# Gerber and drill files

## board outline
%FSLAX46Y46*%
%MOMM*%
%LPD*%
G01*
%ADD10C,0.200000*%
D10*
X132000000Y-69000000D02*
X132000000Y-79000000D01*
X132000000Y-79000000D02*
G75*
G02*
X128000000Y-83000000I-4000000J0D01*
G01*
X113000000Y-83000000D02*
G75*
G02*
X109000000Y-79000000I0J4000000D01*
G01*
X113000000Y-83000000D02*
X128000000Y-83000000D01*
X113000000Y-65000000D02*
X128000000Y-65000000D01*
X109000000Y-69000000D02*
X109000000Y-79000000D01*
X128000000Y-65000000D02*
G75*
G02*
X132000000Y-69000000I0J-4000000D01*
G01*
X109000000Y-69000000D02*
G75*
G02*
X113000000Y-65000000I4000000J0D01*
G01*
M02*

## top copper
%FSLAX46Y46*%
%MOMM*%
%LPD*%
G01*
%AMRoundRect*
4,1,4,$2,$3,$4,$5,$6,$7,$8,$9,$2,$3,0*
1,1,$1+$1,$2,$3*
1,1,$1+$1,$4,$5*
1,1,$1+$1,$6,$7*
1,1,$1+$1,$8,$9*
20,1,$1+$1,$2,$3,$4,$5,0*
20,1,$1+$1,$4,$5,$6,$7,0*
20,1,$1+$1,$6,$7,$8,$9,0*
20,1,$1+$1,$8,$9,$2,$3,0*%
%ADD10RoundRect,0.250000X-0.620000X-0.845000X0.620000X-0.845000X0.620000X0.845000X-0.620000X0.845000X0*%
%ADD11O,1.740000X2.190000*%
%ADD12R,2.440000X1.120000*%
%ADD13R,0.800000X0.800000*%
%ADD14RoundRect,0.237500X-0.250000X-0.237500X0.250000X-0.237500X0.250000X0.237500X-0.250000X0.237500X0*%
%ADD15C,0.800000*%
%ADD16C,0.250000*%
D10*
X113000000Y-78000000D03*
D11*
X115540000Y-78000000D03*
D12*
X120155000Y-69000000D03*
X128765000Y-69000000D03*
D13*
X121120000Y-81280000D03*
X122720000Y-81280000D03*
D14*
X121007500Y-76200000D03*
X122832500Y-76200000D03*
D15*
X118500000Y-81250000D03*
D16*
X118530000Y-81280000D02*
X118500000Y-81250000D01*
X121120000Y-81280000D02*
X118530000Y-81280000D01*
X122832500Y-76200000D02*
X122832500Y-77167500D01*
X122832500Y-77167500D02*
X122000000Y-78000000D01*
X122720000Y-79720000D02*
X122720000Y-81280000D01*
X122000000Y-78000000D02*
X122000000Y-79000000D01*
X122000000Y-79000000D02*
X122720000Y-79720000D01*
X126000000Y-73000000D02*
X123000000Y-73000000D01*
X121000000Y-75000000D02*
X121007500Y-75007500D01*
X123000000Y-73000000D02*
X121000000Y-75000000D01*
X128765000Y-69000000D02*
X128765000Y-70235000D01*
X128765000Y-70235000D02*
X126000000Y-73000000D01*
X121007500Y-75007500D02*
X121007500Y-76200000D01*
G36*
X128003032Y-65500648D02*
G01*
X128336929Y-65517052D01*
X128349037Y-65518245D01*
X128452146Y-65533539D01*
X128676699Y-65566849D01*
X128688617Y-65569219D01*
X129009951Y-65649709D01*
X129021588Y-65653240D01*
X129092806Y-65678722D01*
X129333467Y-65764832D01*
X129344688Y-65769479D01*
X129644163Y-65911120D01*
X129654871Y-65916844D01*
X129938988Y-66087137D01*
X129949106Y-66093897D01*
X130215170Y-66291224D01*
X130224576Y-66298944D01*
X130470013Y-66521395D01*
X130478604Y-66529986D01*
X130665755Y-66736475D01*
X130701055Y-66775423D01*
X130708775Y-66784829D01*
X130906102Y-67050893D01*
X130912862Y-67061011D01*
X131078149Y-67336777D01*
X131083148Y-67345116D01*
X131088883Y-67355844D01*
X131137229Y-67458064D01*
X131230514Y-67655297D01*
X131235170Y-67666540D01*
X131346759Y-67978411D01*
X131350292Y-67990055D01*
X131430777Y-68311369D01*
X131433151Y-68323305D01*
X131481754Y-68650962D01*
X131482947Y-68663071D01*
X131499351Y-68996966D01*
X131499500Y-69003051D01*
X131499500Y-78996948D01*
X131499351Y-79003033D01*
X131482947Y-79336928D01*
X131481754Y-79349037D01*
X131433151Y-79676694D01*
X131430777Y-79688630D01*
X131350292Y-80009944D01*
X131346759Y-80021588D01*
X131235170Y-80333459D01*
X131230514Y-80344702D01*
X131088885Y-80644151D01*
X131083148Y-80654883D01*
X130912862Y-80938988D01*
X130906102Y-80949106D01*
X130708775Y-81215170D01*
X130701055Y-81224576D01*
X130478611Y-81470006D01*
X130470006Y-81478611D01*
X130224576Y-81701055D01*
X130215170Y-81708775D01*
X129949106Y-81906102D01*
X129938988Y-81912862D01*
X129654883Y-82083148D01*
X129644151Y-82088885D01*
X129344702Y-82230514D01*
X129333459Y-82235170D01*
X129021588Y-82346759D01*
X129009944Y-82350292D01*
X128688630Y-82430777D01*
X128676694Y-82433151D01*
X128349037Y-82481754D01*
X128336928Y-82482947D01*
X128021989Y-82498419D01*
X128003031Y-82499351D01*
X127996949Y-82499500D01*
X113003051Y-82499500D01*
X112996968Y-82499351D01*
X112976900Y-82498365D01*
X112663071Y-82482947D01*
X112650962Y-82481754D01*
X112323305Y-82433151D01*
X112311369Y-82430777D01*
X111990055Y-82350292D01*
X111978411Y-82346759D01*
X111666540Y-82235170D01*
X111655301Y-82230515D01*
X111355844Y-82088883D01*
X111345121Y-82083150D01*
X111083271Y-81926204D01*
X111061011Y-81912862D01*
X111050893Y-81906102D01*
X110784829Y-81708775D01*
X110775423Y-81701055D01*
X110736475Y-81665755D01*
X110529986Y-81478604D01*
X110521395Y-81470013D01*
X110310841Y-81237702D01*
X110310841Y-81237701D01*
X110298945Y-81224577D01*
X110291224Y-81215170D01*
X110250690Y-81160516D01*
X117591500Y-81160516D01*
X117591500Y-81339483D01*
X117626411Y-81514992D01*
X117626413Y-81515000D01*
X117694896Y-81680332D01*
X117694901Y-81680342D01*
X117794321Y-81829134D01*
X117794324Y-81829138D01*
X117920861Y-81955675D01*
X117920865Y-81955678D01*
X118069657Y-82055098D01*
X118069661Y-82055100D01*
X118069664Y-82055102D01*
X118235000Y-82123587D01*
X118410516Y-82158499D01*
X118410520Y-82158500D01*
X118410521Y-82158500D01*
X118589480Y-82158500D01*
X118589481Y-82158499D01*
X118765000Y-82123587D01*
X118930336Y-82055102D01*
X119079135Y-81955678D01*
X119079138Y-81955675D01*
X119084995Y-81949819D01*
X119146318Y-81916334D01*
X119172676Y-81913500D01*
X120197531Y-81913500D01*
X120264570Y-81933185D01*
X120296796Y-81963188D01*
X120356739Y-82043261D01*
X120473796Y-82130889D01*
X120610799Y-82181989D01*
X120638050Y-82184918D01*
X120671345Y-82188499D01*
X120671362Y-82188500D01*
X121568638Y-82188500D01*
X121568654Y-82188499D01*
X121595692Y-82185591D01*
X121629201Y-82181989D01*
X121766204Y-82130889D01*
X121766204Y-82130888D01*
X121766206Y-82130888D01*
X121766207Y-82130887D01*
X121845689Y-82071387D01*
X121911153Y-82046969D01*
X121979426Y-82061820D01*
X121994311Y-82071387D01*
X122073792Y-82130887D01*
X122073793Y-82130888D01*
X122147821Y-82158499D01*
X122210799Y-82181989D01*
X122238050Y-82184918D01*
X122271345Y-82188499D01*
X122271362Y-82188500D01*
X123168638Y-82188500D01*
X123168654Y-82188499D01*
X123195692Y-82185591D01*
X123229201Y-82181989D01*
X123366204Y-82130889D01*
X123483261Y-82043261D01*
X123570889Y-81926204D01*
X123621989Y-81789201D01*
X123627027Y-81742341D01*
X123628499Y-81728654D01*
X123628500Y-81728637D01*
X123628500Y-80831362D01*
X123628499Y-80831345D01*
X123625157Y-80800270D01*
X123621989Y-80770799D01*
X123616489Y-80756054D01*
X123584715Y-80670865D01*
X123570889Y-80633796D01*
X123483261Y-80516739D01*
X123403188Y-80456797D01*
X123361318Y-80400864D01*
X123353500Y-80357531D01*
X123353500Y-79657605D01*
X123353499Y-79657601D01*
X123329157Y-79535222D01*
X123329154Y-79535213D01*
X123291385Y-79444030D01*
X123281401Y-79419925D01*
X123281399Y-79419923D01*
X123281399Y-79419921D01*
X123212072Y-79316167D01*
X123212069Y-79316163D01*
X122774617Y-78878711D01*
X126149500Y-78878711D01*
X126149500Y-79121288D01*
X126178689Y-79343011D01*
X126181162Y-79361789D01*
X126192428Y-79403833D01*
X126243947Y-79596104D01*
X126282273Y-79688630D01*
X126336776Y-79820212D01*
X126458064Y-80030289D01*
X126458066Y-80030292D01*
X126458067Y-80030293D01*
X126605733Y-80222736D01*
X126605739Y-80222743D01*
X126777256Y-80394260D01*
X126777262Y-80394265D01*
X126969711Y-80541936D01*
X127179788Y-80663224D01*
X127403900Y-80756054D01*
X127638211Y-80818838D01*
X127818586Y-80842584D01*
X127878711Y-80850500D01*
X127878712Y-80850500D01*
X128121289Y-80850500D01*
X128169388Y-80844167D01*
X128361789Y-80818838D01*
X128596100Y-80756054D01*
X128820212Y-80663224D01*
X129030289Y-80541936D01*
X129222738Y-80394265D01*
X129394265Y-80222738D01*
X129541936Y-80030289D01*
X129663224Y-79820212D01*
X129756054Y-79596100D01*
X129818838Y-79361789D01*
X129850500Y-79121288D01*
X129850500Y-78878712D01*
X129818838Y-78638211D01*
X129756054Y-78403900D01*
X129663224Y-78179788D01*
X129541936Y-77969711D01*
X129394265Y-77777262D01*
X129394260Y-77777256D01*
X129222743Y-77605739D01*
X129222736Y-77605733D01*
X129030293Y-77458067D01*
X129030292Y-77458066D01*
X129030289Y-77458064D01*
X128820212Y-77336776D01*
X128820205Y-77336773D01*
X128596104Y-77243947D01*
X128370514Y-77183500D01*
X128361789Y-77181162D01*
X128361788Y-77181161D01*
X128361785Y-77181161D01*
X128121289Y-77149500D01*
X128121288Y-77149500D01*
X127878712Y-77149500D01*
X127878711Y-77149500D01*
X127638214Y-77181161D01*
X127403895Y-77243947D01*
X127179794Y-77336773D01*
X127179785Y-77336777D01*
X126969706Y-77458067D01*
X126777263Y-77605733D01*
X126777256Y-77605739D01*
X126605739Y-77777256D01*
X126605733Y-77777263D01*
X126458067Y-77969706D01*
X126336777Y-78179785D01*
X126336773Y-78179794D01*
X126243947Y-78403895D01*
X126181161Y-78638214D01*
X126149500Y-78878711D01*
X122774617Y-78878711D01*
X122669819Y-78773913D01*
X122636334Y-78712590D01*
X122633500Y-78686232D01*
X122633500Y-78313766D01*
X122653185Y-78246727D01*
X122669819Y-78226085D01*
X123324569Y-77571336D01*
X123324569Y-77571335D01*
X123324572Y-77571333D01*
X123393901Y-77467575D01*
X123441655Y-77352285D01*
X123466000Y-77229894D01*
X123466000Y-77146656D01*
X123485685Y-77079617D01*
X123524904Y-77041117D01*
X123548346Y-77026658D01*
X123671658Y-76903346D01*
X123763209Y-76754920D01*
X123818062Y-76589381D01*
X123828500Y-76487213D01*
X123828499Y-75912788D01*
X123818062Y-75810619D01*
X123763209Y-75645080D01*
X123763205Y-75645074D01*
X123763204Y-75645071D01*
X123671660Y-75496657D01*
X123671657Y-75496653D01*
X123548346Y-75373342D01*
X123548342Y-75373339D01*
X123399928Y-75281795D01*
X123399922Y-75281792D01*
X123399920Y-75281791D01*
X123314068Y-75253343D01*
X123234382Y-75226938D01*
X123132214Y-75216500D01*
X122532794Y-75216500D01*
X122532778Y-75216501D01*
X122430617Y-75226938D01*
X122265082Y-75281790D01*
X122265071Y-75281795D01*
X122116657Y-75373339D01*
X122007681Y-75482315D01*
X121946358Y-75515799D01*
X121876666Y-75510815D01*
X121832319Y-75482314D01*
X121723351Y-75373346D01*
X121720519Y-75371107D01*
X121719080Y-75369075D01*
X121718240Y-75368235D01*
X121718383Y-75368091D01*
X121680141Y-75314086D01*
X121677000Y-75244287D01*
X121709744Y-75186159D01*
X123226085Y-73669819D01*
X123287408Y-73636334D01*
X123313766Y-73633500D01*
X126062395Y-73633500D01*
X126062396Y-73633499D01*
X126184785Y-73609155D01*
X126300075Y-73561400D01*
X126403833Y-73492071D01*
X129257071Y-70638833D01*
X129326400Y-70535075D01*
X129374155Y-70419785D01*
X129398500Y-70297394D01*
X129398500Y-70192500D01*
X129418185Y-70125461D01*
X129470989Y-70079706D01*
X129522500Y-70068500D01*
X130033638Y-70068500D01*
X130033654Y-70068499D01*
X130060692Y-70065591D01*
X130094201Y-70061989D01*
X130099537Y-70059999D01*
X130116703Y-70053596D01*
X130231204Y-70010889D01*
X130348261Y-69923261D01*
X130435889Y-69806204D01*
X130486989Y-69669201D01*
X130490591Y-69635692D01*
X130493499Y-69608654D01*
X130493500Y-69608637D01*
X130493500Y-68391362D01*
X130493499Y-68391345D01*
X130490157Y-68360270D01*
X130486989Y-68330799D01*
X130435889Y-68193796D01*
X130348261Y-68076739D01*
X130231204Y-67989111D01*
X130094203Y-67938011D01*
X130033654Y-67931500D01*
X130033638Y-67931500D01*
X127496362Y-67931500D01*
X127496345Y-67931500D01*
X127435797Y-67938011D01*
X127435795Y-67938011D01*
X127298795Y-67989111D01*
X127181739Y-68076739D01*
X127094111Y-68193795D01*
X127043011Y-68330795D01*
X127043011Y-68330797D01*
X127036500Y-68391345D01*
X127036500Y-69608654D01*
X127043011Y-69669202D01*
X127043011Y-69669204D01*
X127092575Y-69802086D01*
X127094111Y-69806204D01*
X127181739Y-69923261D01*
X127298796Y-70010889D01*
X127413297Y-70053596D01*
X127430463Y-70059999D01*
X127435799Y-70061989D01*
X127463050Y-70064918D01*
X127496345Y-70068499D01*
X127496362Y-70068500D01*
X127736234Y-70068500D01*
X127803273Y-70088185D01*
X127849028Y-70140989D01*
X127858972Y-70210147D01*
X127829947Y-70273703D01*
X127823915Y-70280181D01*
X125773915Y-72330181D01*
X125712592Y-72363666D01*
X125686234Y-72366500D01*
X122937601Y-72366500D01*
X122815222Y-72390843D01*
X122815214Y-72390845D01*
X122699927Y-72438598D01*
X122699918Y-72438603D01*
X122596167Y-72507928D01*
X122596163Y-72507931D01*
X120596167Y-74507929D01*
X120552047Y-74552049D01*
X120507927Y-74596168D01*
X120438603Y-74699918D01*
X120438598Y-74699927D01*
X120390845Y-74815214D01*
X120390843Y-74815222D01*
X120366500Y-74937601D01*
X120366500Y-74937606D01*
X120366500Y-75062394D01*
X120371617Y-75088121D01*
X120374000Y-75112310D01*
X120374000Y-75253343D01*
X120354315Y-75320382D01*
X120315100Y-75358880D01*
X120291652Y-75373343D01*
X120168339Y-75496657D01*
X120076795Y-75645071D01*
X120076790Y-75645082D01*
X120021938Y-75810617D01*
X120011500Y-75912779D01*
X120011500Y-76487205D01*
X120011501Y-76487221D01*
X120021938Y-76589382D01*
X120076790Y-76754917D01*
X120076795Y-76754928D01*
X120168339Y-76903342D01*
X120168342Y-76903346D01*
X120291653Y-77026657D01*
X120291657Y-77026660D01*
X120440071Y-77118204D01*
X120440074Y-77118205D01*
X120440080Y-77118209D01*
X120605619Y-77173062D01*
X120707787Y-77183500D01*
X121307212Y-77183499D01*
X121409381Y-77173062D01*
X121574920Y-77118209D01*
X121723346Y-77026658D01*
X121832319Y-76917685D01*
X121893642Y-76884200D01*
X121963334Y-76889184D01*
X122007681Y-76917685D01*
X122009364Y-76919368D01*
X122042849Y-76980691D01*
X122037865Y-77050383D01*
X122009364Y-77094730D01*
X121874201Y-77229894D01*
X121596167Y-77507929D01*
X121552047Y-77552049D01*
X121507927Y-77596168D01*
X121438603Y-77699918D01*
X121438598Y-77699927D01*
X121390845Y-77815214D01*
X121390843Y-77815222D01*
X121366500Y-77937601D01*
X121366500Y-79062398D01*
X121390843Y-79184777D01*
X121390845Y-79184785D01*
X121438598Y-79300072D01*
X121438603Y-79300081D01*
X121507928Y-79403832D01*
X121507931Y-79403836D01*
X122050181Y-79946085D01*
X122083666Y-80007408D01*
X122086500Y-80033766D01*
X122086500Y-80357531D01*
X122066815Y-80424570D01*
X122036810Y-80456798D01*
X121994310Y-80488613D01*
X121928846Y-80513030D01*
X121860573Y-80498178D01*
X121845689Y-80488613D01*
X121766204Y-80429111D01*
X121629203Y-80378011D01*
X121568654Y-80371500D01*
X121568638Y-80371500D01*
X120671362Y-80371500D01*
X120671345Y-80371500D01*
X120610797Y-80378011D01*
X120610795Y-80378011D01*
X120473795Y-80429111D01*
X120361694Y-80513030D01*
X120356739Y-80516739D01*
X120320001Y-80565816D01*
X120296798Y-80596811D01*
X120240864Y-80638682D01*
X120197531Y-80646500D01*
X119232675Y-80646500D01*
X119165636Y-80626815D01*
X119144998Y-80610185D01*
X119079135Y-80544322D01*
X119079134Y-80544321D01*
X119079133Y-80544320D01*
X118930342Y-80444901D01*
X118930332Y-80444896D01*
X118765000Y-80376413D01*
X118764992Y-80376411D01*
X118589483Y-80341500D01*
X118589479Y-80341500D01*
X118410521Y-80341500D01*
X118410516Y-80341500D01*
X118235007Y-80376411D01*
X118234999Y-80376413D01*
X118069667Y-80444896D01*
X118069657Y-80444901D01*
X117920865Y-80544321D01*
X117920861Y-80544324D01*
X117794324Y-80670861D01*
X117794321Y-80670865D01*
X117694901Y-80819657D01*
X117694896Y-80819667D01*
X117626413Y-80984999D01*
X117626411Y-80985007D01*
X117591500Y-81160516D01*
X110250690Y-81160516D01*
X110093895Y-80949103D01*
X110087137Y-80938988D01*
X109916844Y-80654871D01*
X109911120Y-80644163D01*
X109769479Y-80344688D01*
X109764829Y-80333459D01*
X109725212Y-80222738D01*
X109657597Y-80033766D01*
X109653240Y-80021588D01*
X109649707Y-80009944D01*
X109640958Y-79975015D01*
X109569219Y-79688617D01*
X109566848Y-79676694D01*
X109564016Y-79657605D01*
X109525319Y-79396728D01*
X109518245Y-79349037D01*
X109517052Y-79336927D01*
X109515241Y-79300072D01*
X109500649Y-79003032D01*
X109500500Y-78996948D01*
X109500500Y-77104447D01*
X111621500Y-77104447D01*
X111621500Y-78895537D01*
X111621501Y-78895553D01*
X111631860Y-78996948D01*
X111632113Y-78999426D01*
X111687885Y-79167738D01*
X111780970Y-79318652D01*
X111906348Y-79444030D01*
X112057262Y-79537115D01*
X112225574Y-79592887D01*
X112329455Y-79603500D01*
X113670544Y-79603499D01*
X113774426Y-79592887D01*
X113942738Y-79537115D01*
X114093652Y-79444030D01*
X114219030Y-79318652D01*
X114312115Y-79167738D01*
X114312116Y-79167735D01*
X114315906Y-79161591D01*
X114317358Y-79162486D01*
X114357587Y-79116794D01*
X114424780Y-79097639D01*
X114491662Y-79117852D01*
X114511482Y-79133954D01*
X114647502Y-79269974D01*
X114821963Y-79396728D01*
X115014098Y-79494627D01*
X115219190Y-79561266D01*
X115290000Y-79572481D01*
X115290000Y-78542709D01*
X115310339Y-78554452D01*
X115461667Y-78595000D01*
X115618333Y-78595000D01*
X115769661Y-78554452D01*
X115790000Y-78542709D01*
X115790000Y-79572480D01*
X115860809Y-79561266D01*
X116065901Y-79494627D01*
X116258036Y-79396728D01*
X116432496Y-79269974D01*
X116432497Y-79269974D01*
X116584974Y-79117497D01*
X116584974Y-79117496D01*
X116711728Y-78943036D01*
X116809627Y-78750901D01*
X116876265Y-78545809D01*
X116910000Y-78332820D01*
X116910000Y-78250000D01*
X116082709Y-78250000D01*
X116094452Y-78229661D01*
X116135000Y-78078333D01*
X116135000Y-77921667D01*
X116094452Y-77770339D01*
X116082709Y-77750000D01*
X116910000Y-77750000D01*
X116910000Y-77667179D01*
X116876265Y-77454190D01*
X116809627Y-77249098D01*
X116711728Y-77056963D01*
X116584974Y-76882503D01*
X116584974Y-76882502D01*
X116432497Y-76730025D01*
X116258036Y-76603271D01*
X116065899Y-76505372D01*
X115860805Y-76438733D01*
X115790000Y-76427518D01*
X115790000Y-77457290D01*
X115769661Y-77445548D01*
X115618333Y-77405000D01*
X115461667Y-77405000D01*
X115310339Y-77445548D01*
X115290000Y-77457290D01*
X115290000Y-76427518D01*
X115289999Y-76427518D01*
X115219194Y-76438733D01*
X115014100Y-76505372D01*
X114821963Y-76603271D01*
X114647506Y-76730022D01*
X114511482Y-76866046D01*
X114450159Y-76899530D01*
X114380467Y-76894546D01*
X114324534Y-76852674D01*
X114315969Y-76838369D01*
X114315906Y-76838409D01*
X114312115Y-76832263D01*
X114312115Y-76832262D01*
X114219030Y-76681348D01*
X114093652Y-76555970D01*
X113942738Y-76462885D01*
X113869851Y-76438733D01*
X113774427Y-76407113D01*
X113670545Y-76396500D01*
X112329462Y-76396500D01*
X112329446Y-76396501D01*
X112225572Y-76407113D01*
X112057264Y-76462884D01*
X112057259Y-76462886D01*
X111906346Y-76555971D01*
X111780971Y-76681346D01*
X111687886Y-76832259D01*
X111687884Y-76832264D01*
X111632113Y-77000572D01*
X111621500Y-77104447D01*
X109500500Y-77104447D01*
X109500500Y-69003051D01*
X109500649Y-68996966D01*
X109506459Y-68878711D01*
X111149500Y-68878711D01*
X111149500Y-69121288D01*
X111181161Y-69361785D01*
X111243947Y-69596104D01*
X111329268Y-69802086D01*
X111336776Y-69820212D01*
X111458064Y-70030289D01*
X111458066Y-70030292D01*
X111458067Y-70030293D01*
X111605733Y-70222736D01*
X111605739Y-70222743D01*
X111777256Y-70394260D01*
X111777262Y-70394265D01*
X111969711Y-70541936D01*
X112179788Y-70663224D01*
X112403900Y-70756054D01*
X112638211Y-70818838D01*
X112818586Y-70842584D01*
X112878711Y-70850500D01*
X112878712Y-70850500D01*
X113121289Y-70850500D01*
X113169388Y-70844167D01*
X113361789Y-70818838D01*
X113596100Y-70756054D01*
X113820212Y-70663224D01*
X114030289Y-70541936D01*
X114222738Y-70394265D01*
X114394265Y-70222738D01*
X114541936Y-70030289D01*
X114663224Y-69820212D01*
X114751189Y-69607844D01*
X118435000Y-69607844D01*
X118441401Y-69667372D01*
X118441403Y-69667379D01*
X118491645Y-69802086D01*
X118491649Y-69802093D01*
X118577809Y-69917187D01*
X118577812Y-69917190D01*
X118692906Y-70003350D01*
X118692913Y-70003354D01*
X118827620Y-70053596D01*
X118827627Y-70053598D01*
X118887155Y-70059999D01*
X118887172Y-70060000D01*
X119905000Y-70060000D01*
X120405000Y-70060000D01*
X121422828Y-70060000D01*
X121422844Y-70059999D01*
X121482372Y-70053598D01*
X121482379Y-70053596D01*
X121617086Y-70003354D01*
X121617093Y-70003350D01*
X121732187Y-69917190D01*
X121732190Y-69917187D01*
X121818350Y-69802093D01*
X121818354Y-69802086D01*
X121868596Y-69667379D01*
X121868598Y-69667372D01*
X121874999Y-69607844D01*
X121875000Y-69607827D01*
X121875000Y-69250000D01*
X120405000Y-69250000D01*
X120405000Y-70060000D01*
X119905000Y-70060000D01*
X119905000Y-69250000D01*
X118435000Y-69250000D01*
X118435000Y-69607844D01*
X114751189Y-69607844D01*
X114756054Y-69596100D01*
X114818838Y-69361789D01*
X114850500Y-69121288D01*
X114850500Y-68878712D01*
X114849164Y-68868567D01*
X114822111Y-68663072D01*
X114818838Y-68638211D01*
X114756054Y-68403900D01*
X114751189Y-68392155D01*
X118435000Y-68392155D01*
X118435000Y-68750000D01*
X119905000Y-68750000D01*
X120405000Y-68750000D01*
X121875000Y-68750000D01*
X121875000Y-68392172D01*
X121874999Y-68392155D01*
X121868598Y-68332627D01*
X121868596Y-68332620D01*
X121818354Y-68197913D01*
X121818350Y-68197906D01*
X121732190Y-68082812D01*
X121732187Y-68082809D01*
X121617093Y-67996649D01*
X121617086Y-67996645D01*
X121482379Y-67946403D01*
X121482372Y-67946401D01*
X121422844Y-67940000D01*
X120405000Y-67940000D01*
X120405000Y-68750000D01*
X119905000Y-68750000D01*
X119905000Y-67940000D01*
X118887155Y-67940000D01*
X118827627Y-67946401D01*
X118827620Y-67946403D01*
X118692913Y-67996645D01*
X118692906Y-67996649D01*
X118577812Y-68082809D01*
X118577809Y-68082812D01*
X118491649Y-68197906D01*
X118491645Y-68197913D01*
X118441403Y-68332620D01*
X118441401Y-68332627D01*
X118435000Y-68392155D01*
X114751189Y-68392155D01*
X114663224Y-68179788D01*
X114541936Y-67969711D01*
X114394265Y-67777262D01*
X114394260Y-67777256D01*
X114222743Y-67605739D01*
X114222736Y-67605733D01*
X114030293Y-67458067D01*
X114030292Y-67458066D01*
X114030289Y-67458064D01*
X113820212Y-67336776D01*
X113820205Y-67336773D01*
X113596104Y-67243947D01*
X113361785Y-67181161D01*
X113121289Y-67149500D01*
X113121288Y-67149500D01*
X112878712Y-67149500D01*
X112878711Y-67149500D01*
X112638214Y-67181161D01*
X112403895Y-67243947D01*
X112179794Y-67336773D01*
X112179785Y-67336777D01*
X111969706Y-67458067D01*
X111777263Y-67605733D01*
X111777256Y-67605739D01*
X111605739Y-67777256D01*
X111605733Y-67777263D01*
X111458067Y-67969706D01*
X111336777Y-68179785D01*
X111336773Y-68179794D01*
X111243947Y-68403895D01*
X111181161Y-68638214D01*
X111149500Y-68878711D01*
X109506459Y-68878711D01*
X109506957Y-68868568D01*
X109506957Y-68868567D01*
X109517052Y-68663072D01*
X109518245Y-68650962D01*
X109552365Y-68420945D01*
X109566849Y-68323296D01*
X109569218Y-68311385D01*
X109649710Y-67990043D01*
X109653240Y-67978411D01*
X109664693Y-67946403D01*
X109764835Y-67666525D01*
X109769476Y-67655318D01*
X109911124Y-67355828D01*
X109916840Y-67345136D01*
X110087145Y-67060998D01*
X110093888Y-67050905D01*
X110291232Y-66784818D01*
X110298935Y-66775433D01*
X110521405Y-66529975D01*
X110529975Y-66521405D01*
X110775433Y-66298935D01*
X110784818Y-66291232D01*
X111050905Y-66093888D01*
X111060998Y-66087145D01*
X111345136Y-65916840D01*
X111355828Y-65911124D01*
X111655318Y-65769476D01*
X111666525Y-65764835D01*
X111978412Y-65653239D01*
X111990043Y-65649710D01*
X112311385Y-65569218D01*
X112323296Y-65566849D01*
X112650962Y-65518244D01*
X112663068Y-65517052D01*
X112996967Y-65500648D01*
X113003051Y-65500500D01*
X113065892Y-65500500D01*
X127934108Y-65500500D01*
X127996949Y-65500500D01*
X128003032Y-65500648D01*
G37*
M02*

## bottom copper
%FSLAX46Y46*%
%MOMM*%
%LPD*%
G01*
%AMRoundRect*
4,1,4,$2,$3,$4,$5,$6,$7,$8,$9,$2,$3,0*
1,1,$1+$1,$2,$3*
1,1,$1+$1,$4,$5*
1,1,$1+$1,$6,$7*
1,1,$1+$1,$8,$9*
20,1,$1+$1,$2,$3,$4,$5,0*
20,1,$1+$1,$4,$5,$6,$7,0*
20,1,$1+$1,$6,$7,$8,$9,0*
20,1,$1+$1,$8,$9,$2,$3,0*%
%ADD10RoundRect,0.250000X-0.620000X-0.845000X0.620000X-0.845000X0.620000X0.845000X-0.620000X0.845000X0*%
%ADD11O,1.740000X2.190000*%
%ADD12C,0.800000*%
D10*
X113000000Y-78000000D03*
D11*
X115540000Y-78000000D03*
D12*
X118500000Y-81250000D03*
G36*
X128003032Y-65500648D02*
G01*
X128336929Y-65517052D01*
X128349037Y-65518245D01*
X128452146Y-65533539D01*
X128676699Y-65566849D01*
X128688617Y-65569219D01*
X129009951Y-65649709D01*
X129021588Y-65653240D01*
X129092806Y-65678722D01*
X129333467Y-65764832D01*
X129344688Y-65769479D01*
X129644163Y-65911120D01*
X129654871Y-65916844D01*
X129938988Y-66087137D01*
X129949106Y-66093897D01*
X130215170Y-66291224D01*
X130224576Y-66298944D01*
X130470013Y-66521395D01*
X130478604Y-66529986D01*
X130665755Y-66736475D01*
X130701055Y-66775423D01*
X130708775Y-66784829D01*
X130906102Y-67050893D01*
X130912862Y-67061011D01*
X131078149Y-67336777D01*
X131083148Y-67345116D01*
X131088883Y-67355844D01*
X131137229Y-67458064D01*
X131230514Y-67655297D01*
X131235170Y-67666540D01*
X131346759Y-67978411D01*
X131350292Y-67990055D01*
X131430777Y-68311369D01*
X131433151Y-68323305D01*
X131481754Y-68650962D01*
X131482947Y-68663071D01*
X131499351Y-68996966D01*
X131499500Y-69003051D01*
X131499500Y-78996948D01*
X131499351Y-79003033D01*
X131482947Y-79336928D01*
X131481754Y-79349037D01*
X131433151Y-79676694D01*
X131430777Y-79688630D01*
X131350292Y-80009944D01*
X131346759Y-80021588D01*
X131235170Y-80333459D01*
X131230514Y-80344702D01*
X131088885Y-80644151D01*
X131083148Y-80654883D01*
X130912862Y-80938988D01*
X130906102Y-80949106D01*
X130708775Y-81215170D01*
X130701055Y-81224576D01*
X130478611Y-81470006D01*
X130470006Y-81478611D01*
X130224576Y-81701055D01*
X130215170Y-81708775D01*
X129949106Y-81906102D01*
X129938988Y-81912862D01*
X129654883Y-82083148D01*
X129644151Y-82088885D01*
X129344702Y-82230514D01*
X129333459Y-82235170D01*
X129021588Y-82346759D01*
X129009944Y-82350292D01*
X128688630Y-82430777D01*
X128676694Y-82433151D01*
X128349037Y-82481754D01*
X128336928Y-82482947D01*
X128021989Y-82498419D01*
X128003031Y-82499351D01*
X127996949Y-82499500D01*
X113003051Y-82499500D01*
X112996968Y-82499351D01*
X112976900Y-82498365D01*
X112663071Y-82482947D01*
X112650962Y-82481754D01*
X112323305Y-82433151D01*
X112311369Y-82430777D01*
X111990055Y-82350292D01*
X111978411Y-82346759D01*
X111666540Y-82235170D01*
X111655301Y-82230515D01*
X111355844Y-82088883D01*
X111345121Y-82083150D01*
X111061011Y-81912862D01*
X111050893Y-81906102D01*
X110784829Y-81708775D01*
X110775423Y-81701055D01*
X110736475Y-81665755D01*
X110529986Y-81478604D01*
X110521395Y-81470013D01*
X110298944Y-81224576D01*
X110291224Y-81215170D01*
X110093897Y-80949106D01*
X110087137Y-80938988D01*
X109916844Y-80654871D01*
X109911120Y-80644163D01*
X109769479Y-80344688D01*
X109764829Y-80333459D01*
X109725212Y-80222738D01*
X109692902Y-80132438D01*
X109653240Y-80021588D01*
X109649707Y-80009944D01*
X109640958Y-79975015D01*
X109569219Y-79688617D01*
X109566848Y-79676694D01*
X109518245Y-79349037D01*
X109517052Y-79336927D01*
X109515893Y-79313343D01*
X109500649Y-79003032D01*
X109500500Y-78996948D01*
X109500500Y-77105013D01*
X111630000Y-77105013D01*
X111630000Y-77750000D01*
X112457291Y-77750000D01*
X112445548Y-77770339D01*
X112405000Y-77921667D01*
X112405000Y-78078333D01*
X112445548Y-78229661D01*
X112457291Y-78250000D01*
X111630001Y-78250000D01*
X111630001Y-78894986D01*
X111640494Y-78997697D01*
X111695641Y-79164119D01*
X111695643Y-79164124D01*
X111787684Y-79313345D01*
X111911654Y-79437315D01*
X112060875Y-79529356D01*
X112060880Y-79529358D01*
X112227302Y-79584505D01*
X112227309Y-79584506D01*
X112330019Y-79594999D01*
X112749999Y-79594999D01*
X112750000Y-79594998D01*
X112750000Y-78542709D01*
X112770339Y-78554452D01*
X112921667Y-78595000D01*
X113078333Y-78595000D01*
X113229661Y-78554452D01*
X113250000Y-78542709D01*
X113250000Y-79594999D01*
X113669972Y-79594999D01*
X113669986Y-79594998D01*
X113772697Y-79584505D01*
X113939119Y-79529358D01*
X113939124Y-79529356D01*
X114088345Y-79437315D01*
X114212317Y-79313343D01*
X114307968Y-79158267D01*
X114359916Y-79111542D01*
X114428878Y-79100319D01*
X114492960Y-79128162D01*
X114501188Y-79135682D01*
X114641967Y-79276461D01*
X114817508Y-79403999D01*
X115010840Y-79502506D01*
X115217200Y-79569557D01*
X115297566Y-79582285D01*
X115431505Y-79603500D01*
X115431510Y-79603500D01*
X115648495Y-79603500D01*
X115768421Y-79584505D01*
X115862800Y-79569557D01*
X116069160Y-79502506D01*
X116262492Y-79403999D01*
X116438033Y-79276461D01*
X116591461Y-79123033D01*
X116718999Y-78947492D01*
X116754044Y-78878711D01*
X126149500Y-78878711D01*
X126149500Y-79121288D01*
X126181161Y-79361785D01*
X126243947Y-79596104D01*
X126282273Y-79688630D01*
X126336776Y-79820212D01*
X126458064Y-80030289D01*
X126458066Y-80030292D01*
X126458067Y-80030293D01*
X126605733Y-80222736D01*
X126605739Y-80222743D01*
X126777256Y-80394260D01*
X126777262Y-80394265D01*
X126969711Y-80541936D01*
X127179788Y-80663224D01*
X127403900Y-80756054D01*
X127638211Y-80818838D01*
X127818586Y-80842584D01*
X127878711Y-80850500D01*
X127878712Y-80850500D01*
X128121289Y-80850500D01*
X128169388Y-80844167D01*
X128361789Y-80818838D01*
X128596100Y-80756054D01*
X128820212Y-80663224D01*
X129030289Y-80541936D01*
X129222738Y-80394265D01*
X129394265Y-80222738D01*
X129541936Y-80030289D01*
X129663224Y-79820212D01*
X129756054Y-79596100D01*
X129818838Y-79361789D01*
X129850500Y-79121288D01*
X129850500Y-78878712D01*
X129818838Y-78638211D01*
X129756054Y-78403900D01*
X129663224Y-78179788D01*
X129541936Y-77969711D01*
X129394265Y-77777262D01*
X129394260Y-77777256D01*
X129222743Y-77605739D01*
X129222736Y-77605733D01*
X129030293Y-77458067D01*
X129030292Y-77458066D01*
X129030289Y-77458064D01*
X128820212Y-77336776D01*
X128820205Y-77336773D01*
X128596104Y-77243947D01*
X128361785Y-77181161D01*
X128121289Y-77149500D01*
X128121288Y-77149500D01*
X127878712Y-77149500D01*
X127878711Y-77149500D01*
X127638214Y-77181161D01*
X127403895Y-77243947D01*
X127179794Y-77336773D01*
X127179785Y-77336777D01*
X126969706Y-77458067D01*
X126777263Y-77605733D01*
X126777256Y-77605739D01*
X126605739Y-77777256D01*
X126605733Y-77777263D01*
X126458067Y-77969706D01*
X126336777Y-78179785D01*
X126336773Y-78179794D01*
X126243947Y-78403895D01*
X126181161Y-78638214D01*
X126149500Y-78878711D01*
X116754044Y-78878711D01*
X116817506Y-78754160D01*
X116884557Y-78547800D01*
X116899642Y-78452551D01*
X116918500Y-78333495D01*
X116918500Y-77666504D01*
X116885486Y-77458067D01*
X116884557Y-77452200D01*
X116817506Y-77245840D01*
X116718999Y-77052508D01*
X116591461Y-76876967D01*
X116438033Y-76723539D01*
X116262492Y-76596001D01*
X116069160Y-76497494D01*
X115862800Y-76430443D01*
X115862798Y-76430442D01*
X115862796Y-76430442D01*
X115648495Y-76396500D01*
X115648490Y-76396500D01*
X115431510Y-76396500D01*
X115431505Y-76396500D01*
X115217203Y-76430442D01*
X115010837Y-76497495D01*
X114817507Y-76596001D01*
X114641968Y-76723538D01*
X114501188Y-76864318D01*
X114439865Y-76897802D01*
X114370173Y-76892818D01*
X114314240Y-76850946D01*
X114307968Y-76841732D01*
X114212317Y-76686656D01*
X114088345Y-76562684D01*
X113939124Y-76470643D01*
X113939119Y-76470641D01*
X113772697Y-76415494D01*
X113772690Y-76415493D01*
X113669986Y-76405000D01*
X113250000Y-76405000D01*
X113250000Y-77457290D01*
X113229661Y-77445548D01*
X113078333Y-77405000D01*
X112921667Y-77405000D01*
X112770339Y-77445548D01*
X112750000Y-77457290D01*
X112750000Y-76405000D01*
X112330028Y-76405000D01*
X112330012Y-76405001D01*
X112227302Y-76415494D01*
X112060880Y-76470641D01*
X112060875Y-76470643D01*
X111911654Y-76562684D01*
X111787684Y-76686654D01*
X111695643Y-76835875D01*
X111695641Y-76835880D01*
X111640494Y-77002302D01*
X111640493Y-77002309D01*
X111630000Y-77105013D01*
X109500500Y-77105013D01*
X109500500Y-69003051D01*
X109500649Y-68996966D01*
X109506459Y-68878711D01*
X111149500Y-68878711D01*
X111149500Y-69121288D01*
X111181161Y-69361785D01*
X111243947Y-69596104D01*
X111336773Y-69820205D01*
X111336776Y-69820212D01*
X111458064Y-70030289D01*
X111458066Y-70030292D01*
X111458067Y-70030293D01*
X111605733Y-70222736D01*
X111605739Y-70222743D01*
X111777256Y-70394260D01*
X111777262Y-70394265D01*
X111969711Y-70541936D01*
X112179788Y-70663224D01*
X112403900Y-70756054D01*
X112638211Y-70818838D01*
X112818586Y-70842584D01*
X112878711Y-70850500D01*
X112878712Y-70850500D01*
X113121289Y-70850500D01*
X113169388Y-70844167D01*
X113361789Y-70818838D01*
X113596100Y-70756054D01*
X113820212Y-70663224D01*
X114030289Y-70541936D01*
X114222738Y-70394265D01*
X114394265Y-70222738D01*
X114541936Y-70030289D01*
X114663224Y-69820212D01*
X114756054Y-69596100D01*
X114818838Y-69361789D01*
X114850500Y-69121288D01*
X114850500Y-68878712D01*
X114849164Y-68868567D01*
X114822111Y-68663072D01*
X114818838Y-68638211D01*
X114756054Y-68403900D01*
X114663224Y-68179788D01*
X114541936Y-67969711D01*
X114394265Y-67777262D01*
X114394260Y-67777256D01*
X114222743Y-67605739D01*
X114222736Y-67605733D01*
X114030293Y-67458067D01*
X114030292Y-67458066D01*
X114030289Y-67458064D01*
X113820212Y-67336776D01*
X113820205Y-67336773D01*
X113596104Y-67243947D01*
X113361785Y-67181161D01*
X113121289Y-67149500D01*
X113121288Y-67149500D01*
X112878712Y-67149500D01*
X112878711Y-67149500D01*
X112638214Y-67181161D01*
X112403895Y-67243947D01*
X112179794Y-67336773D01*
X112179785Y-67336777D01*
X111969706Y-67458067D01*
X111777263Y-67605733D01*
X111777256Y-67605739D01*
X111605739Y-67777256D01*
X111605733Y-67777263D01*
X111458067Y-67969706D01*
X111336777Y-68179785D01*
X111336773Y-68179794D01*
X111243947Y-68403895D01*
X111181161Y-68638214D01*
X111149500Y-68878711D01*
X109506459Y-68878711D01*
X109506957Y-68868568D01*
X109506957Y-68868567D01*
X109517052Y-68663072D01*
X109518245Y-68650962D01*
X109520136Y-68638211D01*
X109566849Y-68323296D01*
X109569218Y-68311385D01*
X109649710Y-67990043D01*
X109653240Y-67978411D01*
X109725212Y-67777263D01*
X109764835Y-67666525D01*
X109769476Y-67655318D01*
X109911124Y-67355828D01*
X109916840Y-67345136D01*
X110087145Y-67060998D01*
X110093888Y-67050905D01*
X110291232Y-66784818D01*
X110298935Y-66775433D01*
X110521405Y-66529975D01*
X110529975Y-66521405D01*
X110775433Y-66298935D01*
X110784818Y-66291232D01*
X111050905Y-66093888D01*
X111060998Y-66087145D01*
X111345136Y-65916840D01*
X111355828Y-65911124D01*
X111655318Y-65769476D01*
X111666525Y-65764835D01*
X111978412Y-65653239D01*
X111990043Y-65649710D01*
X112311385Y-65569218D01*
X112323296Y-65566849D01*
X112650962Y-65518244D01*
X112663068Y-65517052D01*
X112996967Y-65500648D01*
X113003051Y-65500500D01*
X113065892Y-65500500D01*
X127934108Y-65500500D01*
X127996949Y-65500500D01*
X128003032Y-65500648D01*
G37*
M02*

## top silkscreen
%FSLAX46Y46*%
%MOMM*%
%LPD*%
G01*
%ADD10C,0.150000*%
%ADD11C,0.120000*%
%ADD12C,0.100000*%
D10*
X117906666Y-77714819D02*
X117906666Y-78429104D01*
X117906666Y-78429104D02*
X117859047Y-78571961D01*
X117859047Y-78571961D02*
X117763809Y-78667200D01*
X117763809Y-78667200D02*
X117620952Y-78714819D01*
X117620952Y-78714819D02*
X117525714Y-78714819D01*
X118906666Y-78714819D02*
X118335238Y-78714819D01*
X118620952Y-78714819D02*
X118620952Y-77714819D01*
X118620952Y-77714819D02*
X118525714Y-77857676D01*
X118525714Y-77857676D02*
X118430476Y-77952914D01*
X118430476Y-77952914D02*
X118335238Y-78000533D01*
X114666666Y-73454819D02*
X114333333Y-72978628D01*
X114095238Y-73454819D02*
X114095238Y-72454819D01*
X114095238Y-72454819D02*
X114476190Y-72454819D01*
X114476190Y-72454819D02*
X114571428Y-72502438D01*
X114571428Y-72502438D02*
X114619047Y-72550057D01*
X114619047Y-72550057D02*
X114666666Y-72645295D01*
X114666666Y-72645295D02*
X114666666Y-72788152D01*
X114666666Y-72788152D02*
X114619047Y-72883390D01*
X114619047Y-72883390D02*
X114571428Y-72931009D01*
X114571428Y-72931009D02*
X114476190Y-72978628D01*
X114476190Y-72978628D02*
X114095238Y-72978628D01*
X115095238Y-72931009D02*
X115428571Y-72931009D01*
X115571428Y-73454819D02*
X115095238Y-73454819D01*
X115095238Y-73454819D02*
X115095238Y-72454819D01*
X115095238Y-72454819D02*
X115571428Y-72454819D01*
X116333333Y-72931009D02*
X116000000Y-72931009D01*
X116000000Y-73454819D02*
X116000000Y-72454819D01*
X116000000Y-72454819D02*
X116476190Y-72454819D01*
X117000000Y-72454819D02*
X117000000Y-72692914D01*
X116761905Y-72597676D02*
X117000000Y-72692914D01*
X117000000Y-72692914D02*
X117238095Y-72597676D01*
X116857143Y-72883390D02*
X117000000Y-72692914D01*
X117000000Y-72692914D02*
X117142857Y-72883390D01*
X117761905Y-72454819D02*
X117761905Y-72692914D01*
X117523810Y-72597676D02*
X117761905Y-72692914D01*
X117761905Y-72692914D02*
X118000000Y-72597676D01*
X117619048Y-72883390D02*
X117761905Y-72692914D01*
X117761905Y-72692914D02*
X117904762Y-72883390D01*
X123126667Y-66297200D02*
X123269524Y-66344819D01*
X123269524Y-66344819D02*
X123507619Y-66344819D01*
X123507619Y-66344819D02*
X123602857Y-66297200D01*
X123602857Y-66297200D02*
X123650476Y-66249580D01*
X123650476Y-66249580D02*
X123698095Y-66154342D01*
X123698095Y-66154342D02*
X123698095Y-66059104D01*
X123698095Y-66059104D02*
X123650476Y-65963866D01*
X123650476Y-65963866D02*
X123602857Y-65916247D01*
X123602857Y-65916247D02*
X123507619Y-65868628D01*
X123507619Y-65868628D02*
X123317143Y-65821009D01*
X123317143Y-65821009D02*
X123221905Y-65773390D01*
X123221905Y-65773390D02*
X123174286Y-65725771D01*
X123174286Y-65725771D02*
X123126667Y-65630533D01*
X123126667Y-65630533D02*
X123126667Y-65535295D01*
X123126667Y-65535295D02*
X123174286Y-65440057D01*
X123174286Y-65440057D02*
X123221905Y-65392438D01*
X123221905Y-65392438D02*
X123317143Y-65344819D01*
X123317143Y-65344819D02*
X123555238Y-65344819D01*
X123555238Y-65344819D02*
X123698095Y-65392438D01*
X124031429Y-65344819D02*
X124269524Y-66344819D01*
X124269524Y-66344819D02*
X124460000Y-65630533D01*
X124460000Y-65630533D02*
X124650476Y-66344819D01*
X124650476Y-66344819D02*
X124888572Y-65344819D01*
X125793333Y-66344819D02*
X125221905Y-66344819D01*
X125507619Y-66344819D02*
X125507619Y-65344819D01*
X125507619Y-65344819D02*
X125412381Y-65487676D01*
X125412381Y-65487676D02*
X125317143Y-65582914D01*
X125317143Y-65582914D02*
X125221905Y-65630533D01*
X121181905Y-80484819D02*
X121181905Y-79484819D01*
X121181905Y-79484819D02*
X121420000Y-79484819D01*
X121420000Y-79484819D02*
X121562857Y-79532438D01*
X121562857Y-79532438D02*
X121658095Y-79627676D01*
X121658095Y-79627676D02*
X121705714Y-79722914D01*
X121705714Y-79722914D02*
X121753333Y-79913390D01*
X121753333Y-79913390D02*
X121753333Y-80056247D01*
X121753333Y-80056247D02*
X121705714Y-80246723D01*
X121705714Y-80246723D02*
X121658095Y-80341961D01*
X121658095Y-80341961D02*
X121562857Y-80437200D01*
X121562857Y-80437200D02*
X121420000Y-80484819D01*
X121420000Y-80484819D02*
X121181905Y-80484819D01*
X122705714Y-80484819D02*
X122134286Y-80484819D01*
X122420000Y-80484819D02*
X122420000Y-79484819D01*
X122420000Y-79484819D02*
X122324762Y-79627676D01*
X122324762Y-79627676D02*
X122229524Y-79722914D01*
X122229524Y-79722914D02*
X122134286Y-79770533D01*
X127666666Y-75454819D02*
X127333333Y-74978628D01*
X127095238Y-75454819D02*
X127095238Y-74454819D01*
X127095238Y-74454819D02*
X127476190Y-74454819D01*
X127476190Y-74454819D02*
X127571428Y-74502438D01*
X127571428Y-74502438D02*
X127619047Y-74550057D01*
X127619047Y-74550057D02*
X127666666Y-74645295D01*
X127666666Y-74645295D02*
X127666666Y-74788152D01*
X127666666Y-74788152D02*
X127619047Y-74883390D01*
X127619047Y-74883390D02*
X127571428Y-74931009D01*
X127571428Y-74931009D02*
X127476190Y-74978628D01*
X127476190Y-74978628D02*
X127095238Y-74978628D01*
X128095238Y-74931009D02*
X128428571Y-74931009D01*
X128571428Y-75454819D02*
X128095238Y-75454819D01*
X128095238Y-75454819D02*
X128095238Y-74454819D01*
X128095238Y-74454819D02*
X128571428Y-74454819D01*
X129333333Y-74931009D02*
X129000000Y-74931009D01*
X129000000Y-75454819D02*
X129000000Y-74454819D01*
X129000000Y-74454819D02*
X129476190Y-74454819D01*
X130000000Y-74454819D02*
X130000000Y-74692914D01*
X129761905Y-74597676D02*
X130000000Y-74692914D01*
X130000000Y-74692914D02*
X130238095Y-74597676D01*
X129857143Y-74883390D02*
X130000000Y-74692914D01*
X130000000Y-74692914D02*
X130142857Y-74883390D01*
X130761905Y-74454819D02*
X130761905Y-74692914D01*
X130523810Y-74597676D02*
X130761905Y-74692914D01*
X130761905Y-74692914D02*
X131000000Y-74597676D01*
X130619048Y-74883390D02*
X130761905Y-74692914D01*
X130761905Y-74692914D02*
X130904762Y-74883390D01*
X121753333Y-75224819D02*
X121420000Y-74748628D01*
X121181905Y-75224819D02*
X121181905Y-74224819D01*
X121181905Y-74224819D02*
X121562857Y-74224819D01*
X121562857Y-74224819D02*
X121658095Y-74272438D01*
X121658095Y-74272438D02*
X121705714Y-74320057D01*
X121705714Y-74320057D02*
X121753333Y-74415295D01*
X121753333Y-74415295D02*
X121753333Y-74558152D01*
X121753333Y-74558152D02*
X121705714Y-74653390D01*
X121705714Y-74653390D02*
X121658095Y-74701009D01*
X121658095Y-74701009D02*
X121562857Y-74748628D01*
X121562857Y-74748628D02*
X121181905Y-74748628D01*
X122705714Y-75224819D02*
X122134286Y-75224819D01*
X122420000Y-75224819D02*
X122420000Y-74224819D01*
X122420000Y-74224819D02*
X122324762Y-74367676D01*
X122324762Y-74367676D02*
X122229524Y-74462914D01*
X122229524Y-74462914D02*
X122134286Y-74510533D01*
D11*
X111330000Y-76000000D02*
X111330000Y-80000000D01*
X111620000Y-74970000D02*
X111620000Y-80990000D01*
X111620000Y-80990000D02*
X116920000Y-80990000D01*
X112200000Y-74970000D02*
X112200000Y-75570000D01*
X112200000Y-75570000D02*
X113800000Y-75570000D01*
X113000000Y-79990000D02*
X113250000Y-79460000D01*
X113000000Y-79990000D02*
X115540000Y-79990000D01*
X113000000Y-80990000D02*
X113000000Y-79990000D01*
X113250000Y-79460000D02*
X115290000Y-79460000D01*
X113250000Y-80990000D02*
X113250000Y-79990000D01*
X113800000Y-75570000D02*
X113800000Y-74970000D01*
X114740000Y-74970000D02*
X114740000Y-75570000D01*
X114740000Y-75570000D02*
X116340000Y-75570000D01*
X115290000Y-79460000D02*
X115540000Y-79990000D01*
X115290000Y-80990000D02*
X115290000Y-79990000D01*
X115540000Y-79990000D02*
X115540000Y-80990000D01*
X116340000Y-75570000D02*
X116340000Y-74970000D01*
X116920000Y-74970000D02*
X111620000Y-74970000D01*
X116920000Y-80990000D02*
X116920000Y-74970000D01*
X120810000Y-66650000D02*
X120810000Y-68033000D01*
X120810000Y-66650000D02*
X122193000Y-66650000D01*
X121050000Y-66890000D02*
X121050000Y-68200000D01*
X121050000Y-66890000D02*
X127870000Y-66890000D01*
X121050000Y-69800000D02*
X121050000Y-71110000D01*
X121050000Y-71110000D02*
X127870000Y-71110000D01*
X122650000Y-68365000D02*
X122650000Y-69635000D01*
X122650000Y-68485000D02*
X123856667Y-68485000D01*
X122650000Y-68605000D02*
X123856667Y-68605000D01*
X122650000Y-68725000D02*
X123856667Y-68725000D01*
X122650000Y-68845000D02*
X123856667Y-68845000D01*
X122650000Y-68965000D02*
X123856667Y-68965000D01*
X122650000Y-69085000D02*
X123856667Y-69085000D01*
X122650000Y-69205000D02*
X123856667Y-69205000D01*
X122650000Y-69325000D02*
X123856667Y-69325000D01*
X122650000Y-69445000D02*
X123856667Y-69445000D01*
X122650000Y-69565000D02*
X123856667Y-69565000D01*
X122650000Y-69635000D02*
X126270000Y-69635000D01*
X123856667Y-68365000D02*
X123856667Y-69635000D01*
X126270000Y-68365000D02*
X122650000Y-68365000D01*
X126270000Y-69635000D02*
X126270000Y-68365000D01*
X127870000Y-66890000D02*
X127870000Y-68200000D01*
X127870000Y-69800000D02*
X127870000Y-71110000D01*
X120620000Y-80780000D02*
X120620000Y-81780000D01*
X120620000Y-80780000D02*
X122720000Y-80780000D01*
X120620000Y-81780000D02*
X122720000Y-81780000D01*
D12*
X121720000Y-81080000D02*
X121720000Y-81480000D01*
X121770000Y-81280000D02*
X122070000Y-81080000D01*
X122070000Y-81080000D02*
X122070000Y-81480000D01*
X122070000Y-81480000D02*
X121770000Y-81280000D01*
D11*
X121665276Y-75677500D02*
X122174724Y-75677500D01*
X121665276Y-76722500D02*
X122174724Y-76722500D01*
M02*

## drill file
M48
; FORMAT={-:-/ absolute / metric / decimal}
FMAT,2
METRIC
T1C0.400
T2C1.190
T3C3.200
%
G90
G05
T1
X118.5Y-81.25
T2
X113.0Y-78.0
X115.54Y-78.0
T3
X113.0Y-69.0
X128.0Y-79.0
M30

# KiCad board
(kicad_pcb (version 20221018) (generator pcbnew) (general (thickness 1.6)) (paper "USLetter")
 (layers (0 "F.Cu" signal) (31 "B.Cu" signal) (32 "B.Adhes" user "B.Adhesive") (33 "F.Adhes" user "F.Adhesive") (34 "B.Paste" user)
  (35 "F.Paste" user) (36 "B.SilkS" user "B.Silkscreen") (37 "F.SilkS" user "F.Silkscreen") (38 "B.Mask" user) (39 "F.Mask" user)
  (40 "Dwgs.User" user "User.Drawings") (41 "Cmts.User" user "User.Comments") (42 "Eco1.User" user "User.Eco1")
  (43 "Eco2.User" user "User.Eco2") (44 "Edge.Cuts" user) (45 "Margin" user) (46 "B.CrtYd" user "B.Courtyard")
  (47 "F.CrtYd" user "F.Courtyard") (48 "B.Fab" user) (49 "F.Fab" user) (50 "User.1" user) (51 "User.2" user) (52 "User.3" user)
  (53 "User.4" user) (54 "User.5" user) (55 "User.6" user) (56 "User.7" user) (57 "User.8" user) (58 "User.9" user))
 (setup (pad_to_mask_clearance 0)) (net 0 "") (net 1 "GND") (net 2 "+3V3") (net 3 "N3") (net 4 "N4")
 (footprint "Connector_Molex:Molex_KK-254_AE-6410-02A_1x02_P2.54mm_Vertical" (layer "F.Cu") (at 113 78)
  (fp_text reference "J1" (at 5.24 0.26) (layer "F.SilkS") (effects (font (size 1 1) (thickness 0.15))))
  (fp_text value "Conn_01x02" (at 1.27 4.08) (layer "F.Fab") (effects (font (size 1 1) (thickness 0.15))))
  (fp_line (start -1.67 -2) (end -1.67 2) (stroke (width 0.12) (type solid)) (layer "F.SilkS"))
  (fp_line (start -1.38 -3.03) (end -1.38 2.99) (stroke (width 0.12) (type solid)) (layer "F.SilkS"))
  (fp_line (start -1.38 2.99) (end 3.92 2.99) (stroke (width 0.12) (type solid)) (layer "F.SilkS"))
  (fp_line (start -0.8 -3.03) (end -0.8 -2.43) (stroke (width 0.12) (type solid)) (layer "F.SilkS"))
  (fp_line (start -0.8 -2.43) (end 0.8 -2.43) (stroke (width 0.12) (type solid)) (layer "F.SilkS"))
  (fp_line (start 0 1.99) (end 0.25 1.46) (stroke (width 0.12) (type solid)) (layer "F.SilkS"))
  (fp_line (start 0 1.99) (end 2.54 1.99) (stroke (width 0.12) (type solid)) (layer "F.SilkS"))
  (fp_line (start 0 2.99) (end 0 1.99) (stroke (width 0.12) (type solid)) (layer "F.SilkS"))
  (fp_line (start 0.25 1.46) (end 2.29 1.46) (stroke (width 0.12) (type solid)) (layer "F.SilkS"))
  (fp_line (start 0.25 2.99) (end 0.25 1.99) (stroke (width 0.12) (type solid)) (layer "F.SilkS"))
  (fp_line (start 0.8 -2.43) (end 0.8 -3.03) (stroke (width 0.12) (type solid)) (layer "F.SilkS"))
  (fp_line (start 1.74 -3.03) (end 1.74 -2.43) (stroke (width 0.12) (type solid)) (layer "F.SilkS"))
  (fp_line (start 1.74 -2.43) (end 3.34 -2.43) (stroke (width 0.12) (type solid)) (layer "F.SilkS"))
  (fp_line (start 2.29 1.46) (end 2.54 1.99) (stroke (width 0.12) (type solid)) (layer "F.SilkS"))
  (fp_line (start 2.29 2.99) (end 2.29 1.99) (stroke (width 0.12) (type solid)) (layer "F.SilkS"))
  (fp_line (start 2.54 1.99) (end 2.54 2.99) (stroke (width 0.12) (type solid)) (layer "F.SilkS"))
  (fp_line (start 3.34 -2.43) (end 3.34 -3.03) (stroke (width 0.12) (type solid)) (layer "F.SilkS"))
  (fp_line (start 3.92 -3.03) (end -1.38 -3.03) (stroke (width 0.12) (type solid)) (layer "F.SilkS"))
  (fp_line (start 3.92 2.99) (end 3.92 -3.03) (stroke (width 0.12) (type solid)) (layer "F.SilkS"))
  (pad "1" thru_hole roundrect (at 0 0) (size 1.74 2.19) (drill 1.19) (layers "*.Cu" "*.Mask") (roundrect_rratio 0.143678) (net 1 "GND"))
  (pad "2" thru_hole oval (at 2.54 0) (size 1.74 2.19) (drill 1.19) (layers "*.Cu" "*.Mask") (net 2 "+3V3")))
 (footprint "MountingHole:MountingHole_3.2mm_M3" (layer "F.Cu") (at 113 69)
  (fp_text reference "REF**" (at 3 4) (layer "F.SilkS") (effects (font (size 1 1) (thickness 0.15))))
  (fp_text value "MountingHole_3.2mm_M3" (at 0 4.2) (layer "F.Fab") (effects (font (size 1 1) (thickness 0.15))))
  (pad "" np_thru_hole circle (at 0 0) (size 3.2 3.2) (drill 3.2) (layers "F&B.Cu" "*.Mask" "Eco2.User")))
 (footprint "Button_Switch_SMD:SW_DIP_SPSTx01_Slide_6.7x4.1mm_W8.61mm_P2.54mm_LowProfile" (layer "F.Cu") (at 124.46 69)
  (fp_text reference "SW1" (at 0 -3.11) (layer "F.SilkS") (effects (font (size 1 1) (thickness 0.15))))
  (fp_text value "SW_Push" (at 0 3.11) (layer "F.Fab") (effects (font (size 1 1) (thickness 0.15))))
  (fp_line (start -3.65 -2.35) (end -3.65 -0.967) (stroke (width 0.12) (type solid)) (layer "F.SilkS"))
  (fp_line (start -3.65 -2.35) (end -2.267 -2.35) (stroke (width 0.12) (type solid)) (layer "F.SilkS"))
  (fp_line (start -3.41 -2.11) (end -3.41 -0.8) (stroke (width 0.12) (type solid)) (layer "F.SilkS"))
  (fp_line (start -3.41 -2.11) (end 3.41 -2.11) (stroke (width 0.12) (type solid)) (layer "F.SilkS"))
  (fp_line (start -3.41 0.8) (end -3.41 2.11) (stroke (width 0.12) (type solid)) (layer "F.SilkS"))
  (fp_line (start -3.41 2.11) (end 3.41 2.11) (stroke (width 0.12) (type solid)) (layer "F.SilkS"))
  (fp_line (start -1.81 -0.635) (end -1.81 0.635) (stroke (width 0.12) (type solid)) (layer "F.SilkS"))
  (fp_line (start -1.81 -0.515) (end -0.603333 -0.515) (stroke (width 0.12) (type solid)) (layer "F.SilkS"))
  (fp_line (start -1.81 -0.395) (end -0.603333 -0.395) (stroke (width 0.12) (type solid)) (layer "F.SilkS"))
  (fp_line (start -1.81 -0.275) (end -0.603333 -0.275) (stroke (width 0.12) (type solid)) (layer "F.SilkS"))
  (fp_line (start -1.81 -0.155) (end -0.603333 -0.155) (stroke (width 0.12) (type solid)) (layer "F.SilkS"))
  (fp_line (start -1.81 -0.035) (end -0.603333 -0.035) (stroke (width 0.12) (type solid)) (layer "F.SilkS"))
  (fp_line (start -1.81 0.085) (end -0.603333 0.085) (stroke (width 0.12) (type solid)) (layer "F.SilkS"))
  (fp_line (start -1.81 0.205) (end -0.603333 0.205) (stroke (width 0.12) (type solid)) (layer "F.SilkS"))
  (fp_line (start -1.81 0.325) (end -0.603333 0.325) (stroke (width 0.12) (type solid)) (layer "F.SilkS"))
  (fp_line (start -1.81 0.445) (end -0.603333 0.445) (stroke (width 0.12) (type solid)) (layer "F.SilkS"))
  (fp_line (start -1.81 0.565) (end -0.603333 0.565) (stroke (width 0.12) (type solid)) (layer "F.SilkS"))
  (fp_line (start -1.81 0.635) (end 1.81 0.635) (stroke (width 0.12) (type solid)) (layer "F.SilkS"))
  (fp_line (start -0.603333 -0.635) (end -0.603333 0.635) (stroke (width 0.12) (type solid)) (layer "F.SilkS"))
  (fp_line (start 1.81 -0.635) (end -1.81 -0.635) (stroke (width 0.12) (type solid)) (layer "F.SilkS"))
  (fp_line (start 1.81 0.635) (end 1.81 -0.635) (stroke (width 0.12) (type solid)) (layer "F.SilkS"))
  (fp_line (start 3.41 -2.11) (end 3.41 -0.8) (stroke (width 0.12) (type solid)) (layer "F.SilkS"))
  (fp_line (start 3.41 0.8) (end 3.41 2.11) (stroke (width 0.12) (type solid)) (layer "F.SilkS"))
  (pad "1" smd rect (at -4.305 0) (size 2.44 1.12) (layers "F.Cu" "F.Paste" "F.Mask") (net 2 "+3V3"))
  (pad "2" smd rect (at 4.305 0) (size 2.44 1.12) (layers "F.Cu" "F.Paste" "F.Mask") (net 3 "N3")))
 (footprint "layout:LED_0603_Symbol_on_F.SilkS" (layer "F.Cu") (at 121.92 81.28)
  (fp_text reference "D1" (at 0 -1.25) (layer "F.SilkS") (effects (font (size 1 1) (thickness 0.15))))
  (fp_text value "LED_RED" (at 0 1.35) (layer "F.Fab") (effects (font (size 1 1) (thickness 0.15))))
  (fp_line (start -1.3 -0.5) (end -1.3 0.5) (stroke (width 0.12) (type solid)) (layer "F.SilkS"))
  (fp_line (start -1.3 -0.5) (end 0.8 -0.5) (stroke (width 0.12) (type solid)) (layer "F.SilkS"))
  (fp_line (start -1.3 0.5) (end 0.8 0.5) (stroke (width 0.12) (type solid)) (layer "F.SilkS"))
  (fp_line (start -0.2 -0.2) (end -0.2 0.2) (stroke (width 0.1) (type solid)) (layer "F.SilkS"))
  (fp_line (start -0.15 0) (end 0.15 -0.2) (stroke (width 0.1) (type solid)) (layer "F.SilkS"))
  (fp_line (start 0.15 -0.2) (end 0.15 0.2) (stroke (width 0.1) (type solid)) (layer "F.SilkS"))
  (fp_line (start 0.15 0.2) (end -0.15 0) (stroke (width 0.1) (type solid)) (layer "F.SilkS"))
  (pad "1" smd rect (at -0.8 0 180) (size 0.8 0.8) (layers "F.Cu" "F.Paste" "F.Mask") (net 1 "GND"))
  (pad "2" smd rect (at 0.8 0 180) (size 0.8 0.8) (layers "F.Cu" "F.Paste" "F.Mask") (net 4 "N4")))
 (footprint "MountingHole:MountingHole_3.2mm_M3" (layer "F.Cu") (at 128 79 90)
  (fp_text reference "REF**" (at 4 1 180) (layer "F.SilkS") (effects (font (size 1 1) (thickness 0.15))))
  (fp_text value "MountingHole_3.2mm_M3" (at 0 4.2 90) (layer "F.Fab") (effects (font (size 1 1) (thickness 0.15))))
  (pad "" np_thru_hole circle (at 0 0 90) (size 3.2 3.2) (drill 3.2) (layers "F&B.Cu" "*.Mask" "Eco2.User")))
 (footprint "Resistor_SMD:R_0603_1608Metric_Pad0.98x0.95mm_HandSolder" (layer "F.Cu") (at 121.92 76.2)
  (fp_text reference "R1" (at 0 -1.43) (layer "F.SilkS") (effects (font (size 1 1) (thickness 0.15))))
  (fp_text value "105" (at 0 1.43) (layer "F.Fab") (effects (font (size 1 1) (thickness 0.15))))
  (fp_line (start -0.254724 -0.5225) (end 0.254724 -0.5225) (stroke (width 0.12) (type solid)) (layer "F.SilkS"))
  (fp_line (start -0.254724 0.5225) (end 0.254724 0.5225) (stroke (width 0.12) (type solid)) (layer "F.SilkS"))
  (pad "1" smd roundrect (at -0.9125 0) (size 0.975 0.95) (layers "F.Cu" "F.Paste" "F.Mask") (roundrect_rratio 0.25) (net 3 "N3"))
  (pad "2" smd roundrect (at 0.9125 0) (size 0.975 0.95) (layers "F.Cu" "F.Paste" "F.Mask") (roundrect_rratio 0.25) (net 4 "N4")))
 (gr_line (start 132 69) (end 132 79) (stroke (width 0.2) (type default)) (layer "Edge.Cuts"))
 (gr_arc (start 132 79) (mid 130.828427 81.828427) (end 128 83) (stroke (width 0.2) (type default)) (layer "Edge.Cuts"))
 (gr_arc (start 113 83) (mid 110.171573 81.828427) (end 109 79) (stroke (width 0.2) (type default)) (layer "Edge.Cuts"))
 (gr_line (start 113 83) (end 128 83) (stroke (width 0.2) (type default)) (layer "Edge.Cuts"))
 (gr_line (start 113 65) (end 128 65) (stroke (width 0.2) (type default)) (layer "Edge.Cuts"))
 (gr_line (start 109 69) (end 109 79) (stroke (width 0.2) (type default)) (layer "Edge.Cuts"))
 (gr_arc (start 128 65) (mid 130.828427 66.171573) (end 132 69) (stroke (width 0.2) (type default)) (layer "Edge.Cuts"))
 (gr_arc (start 109 69) (mid 110.171573 66.171573) (end 113 65) (stroke (width 0.2) (type default)) (layer "Edge.Cuts"))
 (segment (start 118.53 81.28) (end 118.5 81.25) (width 0.25) (layer "F.Cu") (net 1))
 (segment (start 121.12 81.28) (end 118.53 81.28) (width 0.25) (layer "F.Cu") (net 1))
 (via (at 118.5 81.25) (size 0.8) (drill 0.4) (layers "F.Cu" "B.Cu") (free) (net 1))
 (segment (start 122.8325 76.2) (end 122.8325 77.1675) (width 0.25) (layer "F.Cu") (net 4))
 (segment (start 122.8325 77.1675) (end 122 78) (width 0.25) (layer "F.Cu") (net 4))
 (segment (start 122.72 79.72) (end 122.72 81.28) (width 0.25) (layer "F.Cu") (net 4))
 (segment (start 122 78) (end 122 79) (width 0.25) (layer "F.Cu") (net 4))
 (segment (start 122 79) (end 122.72 79.72) (width 0.25) (layer "F.Cu") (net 4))
 (segment (start 126 73) (end 123 73) (width 0.25) (layer "F.Cu") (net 3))
 (segment (start 121 75) (end 121.0075 75.0075) (width 0.25) (layer "F.Cu") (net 3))
 (segment (start 123 73) (end 121 75) (width 0.25) (layer "F.Cu") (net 3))
 (segment (start 128.765 69) (end 128.765 70.235) (width 0.25) (layer "F.Cu") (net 3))
 (segment (start 128.765 70.235) (end 126 73) (width 0.25) (layer "F.Cu") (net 3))
 (segment (start 121.0075 75.0075) (end 121.0075 76.2) (width 0.25) (layer "F.Cu") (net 3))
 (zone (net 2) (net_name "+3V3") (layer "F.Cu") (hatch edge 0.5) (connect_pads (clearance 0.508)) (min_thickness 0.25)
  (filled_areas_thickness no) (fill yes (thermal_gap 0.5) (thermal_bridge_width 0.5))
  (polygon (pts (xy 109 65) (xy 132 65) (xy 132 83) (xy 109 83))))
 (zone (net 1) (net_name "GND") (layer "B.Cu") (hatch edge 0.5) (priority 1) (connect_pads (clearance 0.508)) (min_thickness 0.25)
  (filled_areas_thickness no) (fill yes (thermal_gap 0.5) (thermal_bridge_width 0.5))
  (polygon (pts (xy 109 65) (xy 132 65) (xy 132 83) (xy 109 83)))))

